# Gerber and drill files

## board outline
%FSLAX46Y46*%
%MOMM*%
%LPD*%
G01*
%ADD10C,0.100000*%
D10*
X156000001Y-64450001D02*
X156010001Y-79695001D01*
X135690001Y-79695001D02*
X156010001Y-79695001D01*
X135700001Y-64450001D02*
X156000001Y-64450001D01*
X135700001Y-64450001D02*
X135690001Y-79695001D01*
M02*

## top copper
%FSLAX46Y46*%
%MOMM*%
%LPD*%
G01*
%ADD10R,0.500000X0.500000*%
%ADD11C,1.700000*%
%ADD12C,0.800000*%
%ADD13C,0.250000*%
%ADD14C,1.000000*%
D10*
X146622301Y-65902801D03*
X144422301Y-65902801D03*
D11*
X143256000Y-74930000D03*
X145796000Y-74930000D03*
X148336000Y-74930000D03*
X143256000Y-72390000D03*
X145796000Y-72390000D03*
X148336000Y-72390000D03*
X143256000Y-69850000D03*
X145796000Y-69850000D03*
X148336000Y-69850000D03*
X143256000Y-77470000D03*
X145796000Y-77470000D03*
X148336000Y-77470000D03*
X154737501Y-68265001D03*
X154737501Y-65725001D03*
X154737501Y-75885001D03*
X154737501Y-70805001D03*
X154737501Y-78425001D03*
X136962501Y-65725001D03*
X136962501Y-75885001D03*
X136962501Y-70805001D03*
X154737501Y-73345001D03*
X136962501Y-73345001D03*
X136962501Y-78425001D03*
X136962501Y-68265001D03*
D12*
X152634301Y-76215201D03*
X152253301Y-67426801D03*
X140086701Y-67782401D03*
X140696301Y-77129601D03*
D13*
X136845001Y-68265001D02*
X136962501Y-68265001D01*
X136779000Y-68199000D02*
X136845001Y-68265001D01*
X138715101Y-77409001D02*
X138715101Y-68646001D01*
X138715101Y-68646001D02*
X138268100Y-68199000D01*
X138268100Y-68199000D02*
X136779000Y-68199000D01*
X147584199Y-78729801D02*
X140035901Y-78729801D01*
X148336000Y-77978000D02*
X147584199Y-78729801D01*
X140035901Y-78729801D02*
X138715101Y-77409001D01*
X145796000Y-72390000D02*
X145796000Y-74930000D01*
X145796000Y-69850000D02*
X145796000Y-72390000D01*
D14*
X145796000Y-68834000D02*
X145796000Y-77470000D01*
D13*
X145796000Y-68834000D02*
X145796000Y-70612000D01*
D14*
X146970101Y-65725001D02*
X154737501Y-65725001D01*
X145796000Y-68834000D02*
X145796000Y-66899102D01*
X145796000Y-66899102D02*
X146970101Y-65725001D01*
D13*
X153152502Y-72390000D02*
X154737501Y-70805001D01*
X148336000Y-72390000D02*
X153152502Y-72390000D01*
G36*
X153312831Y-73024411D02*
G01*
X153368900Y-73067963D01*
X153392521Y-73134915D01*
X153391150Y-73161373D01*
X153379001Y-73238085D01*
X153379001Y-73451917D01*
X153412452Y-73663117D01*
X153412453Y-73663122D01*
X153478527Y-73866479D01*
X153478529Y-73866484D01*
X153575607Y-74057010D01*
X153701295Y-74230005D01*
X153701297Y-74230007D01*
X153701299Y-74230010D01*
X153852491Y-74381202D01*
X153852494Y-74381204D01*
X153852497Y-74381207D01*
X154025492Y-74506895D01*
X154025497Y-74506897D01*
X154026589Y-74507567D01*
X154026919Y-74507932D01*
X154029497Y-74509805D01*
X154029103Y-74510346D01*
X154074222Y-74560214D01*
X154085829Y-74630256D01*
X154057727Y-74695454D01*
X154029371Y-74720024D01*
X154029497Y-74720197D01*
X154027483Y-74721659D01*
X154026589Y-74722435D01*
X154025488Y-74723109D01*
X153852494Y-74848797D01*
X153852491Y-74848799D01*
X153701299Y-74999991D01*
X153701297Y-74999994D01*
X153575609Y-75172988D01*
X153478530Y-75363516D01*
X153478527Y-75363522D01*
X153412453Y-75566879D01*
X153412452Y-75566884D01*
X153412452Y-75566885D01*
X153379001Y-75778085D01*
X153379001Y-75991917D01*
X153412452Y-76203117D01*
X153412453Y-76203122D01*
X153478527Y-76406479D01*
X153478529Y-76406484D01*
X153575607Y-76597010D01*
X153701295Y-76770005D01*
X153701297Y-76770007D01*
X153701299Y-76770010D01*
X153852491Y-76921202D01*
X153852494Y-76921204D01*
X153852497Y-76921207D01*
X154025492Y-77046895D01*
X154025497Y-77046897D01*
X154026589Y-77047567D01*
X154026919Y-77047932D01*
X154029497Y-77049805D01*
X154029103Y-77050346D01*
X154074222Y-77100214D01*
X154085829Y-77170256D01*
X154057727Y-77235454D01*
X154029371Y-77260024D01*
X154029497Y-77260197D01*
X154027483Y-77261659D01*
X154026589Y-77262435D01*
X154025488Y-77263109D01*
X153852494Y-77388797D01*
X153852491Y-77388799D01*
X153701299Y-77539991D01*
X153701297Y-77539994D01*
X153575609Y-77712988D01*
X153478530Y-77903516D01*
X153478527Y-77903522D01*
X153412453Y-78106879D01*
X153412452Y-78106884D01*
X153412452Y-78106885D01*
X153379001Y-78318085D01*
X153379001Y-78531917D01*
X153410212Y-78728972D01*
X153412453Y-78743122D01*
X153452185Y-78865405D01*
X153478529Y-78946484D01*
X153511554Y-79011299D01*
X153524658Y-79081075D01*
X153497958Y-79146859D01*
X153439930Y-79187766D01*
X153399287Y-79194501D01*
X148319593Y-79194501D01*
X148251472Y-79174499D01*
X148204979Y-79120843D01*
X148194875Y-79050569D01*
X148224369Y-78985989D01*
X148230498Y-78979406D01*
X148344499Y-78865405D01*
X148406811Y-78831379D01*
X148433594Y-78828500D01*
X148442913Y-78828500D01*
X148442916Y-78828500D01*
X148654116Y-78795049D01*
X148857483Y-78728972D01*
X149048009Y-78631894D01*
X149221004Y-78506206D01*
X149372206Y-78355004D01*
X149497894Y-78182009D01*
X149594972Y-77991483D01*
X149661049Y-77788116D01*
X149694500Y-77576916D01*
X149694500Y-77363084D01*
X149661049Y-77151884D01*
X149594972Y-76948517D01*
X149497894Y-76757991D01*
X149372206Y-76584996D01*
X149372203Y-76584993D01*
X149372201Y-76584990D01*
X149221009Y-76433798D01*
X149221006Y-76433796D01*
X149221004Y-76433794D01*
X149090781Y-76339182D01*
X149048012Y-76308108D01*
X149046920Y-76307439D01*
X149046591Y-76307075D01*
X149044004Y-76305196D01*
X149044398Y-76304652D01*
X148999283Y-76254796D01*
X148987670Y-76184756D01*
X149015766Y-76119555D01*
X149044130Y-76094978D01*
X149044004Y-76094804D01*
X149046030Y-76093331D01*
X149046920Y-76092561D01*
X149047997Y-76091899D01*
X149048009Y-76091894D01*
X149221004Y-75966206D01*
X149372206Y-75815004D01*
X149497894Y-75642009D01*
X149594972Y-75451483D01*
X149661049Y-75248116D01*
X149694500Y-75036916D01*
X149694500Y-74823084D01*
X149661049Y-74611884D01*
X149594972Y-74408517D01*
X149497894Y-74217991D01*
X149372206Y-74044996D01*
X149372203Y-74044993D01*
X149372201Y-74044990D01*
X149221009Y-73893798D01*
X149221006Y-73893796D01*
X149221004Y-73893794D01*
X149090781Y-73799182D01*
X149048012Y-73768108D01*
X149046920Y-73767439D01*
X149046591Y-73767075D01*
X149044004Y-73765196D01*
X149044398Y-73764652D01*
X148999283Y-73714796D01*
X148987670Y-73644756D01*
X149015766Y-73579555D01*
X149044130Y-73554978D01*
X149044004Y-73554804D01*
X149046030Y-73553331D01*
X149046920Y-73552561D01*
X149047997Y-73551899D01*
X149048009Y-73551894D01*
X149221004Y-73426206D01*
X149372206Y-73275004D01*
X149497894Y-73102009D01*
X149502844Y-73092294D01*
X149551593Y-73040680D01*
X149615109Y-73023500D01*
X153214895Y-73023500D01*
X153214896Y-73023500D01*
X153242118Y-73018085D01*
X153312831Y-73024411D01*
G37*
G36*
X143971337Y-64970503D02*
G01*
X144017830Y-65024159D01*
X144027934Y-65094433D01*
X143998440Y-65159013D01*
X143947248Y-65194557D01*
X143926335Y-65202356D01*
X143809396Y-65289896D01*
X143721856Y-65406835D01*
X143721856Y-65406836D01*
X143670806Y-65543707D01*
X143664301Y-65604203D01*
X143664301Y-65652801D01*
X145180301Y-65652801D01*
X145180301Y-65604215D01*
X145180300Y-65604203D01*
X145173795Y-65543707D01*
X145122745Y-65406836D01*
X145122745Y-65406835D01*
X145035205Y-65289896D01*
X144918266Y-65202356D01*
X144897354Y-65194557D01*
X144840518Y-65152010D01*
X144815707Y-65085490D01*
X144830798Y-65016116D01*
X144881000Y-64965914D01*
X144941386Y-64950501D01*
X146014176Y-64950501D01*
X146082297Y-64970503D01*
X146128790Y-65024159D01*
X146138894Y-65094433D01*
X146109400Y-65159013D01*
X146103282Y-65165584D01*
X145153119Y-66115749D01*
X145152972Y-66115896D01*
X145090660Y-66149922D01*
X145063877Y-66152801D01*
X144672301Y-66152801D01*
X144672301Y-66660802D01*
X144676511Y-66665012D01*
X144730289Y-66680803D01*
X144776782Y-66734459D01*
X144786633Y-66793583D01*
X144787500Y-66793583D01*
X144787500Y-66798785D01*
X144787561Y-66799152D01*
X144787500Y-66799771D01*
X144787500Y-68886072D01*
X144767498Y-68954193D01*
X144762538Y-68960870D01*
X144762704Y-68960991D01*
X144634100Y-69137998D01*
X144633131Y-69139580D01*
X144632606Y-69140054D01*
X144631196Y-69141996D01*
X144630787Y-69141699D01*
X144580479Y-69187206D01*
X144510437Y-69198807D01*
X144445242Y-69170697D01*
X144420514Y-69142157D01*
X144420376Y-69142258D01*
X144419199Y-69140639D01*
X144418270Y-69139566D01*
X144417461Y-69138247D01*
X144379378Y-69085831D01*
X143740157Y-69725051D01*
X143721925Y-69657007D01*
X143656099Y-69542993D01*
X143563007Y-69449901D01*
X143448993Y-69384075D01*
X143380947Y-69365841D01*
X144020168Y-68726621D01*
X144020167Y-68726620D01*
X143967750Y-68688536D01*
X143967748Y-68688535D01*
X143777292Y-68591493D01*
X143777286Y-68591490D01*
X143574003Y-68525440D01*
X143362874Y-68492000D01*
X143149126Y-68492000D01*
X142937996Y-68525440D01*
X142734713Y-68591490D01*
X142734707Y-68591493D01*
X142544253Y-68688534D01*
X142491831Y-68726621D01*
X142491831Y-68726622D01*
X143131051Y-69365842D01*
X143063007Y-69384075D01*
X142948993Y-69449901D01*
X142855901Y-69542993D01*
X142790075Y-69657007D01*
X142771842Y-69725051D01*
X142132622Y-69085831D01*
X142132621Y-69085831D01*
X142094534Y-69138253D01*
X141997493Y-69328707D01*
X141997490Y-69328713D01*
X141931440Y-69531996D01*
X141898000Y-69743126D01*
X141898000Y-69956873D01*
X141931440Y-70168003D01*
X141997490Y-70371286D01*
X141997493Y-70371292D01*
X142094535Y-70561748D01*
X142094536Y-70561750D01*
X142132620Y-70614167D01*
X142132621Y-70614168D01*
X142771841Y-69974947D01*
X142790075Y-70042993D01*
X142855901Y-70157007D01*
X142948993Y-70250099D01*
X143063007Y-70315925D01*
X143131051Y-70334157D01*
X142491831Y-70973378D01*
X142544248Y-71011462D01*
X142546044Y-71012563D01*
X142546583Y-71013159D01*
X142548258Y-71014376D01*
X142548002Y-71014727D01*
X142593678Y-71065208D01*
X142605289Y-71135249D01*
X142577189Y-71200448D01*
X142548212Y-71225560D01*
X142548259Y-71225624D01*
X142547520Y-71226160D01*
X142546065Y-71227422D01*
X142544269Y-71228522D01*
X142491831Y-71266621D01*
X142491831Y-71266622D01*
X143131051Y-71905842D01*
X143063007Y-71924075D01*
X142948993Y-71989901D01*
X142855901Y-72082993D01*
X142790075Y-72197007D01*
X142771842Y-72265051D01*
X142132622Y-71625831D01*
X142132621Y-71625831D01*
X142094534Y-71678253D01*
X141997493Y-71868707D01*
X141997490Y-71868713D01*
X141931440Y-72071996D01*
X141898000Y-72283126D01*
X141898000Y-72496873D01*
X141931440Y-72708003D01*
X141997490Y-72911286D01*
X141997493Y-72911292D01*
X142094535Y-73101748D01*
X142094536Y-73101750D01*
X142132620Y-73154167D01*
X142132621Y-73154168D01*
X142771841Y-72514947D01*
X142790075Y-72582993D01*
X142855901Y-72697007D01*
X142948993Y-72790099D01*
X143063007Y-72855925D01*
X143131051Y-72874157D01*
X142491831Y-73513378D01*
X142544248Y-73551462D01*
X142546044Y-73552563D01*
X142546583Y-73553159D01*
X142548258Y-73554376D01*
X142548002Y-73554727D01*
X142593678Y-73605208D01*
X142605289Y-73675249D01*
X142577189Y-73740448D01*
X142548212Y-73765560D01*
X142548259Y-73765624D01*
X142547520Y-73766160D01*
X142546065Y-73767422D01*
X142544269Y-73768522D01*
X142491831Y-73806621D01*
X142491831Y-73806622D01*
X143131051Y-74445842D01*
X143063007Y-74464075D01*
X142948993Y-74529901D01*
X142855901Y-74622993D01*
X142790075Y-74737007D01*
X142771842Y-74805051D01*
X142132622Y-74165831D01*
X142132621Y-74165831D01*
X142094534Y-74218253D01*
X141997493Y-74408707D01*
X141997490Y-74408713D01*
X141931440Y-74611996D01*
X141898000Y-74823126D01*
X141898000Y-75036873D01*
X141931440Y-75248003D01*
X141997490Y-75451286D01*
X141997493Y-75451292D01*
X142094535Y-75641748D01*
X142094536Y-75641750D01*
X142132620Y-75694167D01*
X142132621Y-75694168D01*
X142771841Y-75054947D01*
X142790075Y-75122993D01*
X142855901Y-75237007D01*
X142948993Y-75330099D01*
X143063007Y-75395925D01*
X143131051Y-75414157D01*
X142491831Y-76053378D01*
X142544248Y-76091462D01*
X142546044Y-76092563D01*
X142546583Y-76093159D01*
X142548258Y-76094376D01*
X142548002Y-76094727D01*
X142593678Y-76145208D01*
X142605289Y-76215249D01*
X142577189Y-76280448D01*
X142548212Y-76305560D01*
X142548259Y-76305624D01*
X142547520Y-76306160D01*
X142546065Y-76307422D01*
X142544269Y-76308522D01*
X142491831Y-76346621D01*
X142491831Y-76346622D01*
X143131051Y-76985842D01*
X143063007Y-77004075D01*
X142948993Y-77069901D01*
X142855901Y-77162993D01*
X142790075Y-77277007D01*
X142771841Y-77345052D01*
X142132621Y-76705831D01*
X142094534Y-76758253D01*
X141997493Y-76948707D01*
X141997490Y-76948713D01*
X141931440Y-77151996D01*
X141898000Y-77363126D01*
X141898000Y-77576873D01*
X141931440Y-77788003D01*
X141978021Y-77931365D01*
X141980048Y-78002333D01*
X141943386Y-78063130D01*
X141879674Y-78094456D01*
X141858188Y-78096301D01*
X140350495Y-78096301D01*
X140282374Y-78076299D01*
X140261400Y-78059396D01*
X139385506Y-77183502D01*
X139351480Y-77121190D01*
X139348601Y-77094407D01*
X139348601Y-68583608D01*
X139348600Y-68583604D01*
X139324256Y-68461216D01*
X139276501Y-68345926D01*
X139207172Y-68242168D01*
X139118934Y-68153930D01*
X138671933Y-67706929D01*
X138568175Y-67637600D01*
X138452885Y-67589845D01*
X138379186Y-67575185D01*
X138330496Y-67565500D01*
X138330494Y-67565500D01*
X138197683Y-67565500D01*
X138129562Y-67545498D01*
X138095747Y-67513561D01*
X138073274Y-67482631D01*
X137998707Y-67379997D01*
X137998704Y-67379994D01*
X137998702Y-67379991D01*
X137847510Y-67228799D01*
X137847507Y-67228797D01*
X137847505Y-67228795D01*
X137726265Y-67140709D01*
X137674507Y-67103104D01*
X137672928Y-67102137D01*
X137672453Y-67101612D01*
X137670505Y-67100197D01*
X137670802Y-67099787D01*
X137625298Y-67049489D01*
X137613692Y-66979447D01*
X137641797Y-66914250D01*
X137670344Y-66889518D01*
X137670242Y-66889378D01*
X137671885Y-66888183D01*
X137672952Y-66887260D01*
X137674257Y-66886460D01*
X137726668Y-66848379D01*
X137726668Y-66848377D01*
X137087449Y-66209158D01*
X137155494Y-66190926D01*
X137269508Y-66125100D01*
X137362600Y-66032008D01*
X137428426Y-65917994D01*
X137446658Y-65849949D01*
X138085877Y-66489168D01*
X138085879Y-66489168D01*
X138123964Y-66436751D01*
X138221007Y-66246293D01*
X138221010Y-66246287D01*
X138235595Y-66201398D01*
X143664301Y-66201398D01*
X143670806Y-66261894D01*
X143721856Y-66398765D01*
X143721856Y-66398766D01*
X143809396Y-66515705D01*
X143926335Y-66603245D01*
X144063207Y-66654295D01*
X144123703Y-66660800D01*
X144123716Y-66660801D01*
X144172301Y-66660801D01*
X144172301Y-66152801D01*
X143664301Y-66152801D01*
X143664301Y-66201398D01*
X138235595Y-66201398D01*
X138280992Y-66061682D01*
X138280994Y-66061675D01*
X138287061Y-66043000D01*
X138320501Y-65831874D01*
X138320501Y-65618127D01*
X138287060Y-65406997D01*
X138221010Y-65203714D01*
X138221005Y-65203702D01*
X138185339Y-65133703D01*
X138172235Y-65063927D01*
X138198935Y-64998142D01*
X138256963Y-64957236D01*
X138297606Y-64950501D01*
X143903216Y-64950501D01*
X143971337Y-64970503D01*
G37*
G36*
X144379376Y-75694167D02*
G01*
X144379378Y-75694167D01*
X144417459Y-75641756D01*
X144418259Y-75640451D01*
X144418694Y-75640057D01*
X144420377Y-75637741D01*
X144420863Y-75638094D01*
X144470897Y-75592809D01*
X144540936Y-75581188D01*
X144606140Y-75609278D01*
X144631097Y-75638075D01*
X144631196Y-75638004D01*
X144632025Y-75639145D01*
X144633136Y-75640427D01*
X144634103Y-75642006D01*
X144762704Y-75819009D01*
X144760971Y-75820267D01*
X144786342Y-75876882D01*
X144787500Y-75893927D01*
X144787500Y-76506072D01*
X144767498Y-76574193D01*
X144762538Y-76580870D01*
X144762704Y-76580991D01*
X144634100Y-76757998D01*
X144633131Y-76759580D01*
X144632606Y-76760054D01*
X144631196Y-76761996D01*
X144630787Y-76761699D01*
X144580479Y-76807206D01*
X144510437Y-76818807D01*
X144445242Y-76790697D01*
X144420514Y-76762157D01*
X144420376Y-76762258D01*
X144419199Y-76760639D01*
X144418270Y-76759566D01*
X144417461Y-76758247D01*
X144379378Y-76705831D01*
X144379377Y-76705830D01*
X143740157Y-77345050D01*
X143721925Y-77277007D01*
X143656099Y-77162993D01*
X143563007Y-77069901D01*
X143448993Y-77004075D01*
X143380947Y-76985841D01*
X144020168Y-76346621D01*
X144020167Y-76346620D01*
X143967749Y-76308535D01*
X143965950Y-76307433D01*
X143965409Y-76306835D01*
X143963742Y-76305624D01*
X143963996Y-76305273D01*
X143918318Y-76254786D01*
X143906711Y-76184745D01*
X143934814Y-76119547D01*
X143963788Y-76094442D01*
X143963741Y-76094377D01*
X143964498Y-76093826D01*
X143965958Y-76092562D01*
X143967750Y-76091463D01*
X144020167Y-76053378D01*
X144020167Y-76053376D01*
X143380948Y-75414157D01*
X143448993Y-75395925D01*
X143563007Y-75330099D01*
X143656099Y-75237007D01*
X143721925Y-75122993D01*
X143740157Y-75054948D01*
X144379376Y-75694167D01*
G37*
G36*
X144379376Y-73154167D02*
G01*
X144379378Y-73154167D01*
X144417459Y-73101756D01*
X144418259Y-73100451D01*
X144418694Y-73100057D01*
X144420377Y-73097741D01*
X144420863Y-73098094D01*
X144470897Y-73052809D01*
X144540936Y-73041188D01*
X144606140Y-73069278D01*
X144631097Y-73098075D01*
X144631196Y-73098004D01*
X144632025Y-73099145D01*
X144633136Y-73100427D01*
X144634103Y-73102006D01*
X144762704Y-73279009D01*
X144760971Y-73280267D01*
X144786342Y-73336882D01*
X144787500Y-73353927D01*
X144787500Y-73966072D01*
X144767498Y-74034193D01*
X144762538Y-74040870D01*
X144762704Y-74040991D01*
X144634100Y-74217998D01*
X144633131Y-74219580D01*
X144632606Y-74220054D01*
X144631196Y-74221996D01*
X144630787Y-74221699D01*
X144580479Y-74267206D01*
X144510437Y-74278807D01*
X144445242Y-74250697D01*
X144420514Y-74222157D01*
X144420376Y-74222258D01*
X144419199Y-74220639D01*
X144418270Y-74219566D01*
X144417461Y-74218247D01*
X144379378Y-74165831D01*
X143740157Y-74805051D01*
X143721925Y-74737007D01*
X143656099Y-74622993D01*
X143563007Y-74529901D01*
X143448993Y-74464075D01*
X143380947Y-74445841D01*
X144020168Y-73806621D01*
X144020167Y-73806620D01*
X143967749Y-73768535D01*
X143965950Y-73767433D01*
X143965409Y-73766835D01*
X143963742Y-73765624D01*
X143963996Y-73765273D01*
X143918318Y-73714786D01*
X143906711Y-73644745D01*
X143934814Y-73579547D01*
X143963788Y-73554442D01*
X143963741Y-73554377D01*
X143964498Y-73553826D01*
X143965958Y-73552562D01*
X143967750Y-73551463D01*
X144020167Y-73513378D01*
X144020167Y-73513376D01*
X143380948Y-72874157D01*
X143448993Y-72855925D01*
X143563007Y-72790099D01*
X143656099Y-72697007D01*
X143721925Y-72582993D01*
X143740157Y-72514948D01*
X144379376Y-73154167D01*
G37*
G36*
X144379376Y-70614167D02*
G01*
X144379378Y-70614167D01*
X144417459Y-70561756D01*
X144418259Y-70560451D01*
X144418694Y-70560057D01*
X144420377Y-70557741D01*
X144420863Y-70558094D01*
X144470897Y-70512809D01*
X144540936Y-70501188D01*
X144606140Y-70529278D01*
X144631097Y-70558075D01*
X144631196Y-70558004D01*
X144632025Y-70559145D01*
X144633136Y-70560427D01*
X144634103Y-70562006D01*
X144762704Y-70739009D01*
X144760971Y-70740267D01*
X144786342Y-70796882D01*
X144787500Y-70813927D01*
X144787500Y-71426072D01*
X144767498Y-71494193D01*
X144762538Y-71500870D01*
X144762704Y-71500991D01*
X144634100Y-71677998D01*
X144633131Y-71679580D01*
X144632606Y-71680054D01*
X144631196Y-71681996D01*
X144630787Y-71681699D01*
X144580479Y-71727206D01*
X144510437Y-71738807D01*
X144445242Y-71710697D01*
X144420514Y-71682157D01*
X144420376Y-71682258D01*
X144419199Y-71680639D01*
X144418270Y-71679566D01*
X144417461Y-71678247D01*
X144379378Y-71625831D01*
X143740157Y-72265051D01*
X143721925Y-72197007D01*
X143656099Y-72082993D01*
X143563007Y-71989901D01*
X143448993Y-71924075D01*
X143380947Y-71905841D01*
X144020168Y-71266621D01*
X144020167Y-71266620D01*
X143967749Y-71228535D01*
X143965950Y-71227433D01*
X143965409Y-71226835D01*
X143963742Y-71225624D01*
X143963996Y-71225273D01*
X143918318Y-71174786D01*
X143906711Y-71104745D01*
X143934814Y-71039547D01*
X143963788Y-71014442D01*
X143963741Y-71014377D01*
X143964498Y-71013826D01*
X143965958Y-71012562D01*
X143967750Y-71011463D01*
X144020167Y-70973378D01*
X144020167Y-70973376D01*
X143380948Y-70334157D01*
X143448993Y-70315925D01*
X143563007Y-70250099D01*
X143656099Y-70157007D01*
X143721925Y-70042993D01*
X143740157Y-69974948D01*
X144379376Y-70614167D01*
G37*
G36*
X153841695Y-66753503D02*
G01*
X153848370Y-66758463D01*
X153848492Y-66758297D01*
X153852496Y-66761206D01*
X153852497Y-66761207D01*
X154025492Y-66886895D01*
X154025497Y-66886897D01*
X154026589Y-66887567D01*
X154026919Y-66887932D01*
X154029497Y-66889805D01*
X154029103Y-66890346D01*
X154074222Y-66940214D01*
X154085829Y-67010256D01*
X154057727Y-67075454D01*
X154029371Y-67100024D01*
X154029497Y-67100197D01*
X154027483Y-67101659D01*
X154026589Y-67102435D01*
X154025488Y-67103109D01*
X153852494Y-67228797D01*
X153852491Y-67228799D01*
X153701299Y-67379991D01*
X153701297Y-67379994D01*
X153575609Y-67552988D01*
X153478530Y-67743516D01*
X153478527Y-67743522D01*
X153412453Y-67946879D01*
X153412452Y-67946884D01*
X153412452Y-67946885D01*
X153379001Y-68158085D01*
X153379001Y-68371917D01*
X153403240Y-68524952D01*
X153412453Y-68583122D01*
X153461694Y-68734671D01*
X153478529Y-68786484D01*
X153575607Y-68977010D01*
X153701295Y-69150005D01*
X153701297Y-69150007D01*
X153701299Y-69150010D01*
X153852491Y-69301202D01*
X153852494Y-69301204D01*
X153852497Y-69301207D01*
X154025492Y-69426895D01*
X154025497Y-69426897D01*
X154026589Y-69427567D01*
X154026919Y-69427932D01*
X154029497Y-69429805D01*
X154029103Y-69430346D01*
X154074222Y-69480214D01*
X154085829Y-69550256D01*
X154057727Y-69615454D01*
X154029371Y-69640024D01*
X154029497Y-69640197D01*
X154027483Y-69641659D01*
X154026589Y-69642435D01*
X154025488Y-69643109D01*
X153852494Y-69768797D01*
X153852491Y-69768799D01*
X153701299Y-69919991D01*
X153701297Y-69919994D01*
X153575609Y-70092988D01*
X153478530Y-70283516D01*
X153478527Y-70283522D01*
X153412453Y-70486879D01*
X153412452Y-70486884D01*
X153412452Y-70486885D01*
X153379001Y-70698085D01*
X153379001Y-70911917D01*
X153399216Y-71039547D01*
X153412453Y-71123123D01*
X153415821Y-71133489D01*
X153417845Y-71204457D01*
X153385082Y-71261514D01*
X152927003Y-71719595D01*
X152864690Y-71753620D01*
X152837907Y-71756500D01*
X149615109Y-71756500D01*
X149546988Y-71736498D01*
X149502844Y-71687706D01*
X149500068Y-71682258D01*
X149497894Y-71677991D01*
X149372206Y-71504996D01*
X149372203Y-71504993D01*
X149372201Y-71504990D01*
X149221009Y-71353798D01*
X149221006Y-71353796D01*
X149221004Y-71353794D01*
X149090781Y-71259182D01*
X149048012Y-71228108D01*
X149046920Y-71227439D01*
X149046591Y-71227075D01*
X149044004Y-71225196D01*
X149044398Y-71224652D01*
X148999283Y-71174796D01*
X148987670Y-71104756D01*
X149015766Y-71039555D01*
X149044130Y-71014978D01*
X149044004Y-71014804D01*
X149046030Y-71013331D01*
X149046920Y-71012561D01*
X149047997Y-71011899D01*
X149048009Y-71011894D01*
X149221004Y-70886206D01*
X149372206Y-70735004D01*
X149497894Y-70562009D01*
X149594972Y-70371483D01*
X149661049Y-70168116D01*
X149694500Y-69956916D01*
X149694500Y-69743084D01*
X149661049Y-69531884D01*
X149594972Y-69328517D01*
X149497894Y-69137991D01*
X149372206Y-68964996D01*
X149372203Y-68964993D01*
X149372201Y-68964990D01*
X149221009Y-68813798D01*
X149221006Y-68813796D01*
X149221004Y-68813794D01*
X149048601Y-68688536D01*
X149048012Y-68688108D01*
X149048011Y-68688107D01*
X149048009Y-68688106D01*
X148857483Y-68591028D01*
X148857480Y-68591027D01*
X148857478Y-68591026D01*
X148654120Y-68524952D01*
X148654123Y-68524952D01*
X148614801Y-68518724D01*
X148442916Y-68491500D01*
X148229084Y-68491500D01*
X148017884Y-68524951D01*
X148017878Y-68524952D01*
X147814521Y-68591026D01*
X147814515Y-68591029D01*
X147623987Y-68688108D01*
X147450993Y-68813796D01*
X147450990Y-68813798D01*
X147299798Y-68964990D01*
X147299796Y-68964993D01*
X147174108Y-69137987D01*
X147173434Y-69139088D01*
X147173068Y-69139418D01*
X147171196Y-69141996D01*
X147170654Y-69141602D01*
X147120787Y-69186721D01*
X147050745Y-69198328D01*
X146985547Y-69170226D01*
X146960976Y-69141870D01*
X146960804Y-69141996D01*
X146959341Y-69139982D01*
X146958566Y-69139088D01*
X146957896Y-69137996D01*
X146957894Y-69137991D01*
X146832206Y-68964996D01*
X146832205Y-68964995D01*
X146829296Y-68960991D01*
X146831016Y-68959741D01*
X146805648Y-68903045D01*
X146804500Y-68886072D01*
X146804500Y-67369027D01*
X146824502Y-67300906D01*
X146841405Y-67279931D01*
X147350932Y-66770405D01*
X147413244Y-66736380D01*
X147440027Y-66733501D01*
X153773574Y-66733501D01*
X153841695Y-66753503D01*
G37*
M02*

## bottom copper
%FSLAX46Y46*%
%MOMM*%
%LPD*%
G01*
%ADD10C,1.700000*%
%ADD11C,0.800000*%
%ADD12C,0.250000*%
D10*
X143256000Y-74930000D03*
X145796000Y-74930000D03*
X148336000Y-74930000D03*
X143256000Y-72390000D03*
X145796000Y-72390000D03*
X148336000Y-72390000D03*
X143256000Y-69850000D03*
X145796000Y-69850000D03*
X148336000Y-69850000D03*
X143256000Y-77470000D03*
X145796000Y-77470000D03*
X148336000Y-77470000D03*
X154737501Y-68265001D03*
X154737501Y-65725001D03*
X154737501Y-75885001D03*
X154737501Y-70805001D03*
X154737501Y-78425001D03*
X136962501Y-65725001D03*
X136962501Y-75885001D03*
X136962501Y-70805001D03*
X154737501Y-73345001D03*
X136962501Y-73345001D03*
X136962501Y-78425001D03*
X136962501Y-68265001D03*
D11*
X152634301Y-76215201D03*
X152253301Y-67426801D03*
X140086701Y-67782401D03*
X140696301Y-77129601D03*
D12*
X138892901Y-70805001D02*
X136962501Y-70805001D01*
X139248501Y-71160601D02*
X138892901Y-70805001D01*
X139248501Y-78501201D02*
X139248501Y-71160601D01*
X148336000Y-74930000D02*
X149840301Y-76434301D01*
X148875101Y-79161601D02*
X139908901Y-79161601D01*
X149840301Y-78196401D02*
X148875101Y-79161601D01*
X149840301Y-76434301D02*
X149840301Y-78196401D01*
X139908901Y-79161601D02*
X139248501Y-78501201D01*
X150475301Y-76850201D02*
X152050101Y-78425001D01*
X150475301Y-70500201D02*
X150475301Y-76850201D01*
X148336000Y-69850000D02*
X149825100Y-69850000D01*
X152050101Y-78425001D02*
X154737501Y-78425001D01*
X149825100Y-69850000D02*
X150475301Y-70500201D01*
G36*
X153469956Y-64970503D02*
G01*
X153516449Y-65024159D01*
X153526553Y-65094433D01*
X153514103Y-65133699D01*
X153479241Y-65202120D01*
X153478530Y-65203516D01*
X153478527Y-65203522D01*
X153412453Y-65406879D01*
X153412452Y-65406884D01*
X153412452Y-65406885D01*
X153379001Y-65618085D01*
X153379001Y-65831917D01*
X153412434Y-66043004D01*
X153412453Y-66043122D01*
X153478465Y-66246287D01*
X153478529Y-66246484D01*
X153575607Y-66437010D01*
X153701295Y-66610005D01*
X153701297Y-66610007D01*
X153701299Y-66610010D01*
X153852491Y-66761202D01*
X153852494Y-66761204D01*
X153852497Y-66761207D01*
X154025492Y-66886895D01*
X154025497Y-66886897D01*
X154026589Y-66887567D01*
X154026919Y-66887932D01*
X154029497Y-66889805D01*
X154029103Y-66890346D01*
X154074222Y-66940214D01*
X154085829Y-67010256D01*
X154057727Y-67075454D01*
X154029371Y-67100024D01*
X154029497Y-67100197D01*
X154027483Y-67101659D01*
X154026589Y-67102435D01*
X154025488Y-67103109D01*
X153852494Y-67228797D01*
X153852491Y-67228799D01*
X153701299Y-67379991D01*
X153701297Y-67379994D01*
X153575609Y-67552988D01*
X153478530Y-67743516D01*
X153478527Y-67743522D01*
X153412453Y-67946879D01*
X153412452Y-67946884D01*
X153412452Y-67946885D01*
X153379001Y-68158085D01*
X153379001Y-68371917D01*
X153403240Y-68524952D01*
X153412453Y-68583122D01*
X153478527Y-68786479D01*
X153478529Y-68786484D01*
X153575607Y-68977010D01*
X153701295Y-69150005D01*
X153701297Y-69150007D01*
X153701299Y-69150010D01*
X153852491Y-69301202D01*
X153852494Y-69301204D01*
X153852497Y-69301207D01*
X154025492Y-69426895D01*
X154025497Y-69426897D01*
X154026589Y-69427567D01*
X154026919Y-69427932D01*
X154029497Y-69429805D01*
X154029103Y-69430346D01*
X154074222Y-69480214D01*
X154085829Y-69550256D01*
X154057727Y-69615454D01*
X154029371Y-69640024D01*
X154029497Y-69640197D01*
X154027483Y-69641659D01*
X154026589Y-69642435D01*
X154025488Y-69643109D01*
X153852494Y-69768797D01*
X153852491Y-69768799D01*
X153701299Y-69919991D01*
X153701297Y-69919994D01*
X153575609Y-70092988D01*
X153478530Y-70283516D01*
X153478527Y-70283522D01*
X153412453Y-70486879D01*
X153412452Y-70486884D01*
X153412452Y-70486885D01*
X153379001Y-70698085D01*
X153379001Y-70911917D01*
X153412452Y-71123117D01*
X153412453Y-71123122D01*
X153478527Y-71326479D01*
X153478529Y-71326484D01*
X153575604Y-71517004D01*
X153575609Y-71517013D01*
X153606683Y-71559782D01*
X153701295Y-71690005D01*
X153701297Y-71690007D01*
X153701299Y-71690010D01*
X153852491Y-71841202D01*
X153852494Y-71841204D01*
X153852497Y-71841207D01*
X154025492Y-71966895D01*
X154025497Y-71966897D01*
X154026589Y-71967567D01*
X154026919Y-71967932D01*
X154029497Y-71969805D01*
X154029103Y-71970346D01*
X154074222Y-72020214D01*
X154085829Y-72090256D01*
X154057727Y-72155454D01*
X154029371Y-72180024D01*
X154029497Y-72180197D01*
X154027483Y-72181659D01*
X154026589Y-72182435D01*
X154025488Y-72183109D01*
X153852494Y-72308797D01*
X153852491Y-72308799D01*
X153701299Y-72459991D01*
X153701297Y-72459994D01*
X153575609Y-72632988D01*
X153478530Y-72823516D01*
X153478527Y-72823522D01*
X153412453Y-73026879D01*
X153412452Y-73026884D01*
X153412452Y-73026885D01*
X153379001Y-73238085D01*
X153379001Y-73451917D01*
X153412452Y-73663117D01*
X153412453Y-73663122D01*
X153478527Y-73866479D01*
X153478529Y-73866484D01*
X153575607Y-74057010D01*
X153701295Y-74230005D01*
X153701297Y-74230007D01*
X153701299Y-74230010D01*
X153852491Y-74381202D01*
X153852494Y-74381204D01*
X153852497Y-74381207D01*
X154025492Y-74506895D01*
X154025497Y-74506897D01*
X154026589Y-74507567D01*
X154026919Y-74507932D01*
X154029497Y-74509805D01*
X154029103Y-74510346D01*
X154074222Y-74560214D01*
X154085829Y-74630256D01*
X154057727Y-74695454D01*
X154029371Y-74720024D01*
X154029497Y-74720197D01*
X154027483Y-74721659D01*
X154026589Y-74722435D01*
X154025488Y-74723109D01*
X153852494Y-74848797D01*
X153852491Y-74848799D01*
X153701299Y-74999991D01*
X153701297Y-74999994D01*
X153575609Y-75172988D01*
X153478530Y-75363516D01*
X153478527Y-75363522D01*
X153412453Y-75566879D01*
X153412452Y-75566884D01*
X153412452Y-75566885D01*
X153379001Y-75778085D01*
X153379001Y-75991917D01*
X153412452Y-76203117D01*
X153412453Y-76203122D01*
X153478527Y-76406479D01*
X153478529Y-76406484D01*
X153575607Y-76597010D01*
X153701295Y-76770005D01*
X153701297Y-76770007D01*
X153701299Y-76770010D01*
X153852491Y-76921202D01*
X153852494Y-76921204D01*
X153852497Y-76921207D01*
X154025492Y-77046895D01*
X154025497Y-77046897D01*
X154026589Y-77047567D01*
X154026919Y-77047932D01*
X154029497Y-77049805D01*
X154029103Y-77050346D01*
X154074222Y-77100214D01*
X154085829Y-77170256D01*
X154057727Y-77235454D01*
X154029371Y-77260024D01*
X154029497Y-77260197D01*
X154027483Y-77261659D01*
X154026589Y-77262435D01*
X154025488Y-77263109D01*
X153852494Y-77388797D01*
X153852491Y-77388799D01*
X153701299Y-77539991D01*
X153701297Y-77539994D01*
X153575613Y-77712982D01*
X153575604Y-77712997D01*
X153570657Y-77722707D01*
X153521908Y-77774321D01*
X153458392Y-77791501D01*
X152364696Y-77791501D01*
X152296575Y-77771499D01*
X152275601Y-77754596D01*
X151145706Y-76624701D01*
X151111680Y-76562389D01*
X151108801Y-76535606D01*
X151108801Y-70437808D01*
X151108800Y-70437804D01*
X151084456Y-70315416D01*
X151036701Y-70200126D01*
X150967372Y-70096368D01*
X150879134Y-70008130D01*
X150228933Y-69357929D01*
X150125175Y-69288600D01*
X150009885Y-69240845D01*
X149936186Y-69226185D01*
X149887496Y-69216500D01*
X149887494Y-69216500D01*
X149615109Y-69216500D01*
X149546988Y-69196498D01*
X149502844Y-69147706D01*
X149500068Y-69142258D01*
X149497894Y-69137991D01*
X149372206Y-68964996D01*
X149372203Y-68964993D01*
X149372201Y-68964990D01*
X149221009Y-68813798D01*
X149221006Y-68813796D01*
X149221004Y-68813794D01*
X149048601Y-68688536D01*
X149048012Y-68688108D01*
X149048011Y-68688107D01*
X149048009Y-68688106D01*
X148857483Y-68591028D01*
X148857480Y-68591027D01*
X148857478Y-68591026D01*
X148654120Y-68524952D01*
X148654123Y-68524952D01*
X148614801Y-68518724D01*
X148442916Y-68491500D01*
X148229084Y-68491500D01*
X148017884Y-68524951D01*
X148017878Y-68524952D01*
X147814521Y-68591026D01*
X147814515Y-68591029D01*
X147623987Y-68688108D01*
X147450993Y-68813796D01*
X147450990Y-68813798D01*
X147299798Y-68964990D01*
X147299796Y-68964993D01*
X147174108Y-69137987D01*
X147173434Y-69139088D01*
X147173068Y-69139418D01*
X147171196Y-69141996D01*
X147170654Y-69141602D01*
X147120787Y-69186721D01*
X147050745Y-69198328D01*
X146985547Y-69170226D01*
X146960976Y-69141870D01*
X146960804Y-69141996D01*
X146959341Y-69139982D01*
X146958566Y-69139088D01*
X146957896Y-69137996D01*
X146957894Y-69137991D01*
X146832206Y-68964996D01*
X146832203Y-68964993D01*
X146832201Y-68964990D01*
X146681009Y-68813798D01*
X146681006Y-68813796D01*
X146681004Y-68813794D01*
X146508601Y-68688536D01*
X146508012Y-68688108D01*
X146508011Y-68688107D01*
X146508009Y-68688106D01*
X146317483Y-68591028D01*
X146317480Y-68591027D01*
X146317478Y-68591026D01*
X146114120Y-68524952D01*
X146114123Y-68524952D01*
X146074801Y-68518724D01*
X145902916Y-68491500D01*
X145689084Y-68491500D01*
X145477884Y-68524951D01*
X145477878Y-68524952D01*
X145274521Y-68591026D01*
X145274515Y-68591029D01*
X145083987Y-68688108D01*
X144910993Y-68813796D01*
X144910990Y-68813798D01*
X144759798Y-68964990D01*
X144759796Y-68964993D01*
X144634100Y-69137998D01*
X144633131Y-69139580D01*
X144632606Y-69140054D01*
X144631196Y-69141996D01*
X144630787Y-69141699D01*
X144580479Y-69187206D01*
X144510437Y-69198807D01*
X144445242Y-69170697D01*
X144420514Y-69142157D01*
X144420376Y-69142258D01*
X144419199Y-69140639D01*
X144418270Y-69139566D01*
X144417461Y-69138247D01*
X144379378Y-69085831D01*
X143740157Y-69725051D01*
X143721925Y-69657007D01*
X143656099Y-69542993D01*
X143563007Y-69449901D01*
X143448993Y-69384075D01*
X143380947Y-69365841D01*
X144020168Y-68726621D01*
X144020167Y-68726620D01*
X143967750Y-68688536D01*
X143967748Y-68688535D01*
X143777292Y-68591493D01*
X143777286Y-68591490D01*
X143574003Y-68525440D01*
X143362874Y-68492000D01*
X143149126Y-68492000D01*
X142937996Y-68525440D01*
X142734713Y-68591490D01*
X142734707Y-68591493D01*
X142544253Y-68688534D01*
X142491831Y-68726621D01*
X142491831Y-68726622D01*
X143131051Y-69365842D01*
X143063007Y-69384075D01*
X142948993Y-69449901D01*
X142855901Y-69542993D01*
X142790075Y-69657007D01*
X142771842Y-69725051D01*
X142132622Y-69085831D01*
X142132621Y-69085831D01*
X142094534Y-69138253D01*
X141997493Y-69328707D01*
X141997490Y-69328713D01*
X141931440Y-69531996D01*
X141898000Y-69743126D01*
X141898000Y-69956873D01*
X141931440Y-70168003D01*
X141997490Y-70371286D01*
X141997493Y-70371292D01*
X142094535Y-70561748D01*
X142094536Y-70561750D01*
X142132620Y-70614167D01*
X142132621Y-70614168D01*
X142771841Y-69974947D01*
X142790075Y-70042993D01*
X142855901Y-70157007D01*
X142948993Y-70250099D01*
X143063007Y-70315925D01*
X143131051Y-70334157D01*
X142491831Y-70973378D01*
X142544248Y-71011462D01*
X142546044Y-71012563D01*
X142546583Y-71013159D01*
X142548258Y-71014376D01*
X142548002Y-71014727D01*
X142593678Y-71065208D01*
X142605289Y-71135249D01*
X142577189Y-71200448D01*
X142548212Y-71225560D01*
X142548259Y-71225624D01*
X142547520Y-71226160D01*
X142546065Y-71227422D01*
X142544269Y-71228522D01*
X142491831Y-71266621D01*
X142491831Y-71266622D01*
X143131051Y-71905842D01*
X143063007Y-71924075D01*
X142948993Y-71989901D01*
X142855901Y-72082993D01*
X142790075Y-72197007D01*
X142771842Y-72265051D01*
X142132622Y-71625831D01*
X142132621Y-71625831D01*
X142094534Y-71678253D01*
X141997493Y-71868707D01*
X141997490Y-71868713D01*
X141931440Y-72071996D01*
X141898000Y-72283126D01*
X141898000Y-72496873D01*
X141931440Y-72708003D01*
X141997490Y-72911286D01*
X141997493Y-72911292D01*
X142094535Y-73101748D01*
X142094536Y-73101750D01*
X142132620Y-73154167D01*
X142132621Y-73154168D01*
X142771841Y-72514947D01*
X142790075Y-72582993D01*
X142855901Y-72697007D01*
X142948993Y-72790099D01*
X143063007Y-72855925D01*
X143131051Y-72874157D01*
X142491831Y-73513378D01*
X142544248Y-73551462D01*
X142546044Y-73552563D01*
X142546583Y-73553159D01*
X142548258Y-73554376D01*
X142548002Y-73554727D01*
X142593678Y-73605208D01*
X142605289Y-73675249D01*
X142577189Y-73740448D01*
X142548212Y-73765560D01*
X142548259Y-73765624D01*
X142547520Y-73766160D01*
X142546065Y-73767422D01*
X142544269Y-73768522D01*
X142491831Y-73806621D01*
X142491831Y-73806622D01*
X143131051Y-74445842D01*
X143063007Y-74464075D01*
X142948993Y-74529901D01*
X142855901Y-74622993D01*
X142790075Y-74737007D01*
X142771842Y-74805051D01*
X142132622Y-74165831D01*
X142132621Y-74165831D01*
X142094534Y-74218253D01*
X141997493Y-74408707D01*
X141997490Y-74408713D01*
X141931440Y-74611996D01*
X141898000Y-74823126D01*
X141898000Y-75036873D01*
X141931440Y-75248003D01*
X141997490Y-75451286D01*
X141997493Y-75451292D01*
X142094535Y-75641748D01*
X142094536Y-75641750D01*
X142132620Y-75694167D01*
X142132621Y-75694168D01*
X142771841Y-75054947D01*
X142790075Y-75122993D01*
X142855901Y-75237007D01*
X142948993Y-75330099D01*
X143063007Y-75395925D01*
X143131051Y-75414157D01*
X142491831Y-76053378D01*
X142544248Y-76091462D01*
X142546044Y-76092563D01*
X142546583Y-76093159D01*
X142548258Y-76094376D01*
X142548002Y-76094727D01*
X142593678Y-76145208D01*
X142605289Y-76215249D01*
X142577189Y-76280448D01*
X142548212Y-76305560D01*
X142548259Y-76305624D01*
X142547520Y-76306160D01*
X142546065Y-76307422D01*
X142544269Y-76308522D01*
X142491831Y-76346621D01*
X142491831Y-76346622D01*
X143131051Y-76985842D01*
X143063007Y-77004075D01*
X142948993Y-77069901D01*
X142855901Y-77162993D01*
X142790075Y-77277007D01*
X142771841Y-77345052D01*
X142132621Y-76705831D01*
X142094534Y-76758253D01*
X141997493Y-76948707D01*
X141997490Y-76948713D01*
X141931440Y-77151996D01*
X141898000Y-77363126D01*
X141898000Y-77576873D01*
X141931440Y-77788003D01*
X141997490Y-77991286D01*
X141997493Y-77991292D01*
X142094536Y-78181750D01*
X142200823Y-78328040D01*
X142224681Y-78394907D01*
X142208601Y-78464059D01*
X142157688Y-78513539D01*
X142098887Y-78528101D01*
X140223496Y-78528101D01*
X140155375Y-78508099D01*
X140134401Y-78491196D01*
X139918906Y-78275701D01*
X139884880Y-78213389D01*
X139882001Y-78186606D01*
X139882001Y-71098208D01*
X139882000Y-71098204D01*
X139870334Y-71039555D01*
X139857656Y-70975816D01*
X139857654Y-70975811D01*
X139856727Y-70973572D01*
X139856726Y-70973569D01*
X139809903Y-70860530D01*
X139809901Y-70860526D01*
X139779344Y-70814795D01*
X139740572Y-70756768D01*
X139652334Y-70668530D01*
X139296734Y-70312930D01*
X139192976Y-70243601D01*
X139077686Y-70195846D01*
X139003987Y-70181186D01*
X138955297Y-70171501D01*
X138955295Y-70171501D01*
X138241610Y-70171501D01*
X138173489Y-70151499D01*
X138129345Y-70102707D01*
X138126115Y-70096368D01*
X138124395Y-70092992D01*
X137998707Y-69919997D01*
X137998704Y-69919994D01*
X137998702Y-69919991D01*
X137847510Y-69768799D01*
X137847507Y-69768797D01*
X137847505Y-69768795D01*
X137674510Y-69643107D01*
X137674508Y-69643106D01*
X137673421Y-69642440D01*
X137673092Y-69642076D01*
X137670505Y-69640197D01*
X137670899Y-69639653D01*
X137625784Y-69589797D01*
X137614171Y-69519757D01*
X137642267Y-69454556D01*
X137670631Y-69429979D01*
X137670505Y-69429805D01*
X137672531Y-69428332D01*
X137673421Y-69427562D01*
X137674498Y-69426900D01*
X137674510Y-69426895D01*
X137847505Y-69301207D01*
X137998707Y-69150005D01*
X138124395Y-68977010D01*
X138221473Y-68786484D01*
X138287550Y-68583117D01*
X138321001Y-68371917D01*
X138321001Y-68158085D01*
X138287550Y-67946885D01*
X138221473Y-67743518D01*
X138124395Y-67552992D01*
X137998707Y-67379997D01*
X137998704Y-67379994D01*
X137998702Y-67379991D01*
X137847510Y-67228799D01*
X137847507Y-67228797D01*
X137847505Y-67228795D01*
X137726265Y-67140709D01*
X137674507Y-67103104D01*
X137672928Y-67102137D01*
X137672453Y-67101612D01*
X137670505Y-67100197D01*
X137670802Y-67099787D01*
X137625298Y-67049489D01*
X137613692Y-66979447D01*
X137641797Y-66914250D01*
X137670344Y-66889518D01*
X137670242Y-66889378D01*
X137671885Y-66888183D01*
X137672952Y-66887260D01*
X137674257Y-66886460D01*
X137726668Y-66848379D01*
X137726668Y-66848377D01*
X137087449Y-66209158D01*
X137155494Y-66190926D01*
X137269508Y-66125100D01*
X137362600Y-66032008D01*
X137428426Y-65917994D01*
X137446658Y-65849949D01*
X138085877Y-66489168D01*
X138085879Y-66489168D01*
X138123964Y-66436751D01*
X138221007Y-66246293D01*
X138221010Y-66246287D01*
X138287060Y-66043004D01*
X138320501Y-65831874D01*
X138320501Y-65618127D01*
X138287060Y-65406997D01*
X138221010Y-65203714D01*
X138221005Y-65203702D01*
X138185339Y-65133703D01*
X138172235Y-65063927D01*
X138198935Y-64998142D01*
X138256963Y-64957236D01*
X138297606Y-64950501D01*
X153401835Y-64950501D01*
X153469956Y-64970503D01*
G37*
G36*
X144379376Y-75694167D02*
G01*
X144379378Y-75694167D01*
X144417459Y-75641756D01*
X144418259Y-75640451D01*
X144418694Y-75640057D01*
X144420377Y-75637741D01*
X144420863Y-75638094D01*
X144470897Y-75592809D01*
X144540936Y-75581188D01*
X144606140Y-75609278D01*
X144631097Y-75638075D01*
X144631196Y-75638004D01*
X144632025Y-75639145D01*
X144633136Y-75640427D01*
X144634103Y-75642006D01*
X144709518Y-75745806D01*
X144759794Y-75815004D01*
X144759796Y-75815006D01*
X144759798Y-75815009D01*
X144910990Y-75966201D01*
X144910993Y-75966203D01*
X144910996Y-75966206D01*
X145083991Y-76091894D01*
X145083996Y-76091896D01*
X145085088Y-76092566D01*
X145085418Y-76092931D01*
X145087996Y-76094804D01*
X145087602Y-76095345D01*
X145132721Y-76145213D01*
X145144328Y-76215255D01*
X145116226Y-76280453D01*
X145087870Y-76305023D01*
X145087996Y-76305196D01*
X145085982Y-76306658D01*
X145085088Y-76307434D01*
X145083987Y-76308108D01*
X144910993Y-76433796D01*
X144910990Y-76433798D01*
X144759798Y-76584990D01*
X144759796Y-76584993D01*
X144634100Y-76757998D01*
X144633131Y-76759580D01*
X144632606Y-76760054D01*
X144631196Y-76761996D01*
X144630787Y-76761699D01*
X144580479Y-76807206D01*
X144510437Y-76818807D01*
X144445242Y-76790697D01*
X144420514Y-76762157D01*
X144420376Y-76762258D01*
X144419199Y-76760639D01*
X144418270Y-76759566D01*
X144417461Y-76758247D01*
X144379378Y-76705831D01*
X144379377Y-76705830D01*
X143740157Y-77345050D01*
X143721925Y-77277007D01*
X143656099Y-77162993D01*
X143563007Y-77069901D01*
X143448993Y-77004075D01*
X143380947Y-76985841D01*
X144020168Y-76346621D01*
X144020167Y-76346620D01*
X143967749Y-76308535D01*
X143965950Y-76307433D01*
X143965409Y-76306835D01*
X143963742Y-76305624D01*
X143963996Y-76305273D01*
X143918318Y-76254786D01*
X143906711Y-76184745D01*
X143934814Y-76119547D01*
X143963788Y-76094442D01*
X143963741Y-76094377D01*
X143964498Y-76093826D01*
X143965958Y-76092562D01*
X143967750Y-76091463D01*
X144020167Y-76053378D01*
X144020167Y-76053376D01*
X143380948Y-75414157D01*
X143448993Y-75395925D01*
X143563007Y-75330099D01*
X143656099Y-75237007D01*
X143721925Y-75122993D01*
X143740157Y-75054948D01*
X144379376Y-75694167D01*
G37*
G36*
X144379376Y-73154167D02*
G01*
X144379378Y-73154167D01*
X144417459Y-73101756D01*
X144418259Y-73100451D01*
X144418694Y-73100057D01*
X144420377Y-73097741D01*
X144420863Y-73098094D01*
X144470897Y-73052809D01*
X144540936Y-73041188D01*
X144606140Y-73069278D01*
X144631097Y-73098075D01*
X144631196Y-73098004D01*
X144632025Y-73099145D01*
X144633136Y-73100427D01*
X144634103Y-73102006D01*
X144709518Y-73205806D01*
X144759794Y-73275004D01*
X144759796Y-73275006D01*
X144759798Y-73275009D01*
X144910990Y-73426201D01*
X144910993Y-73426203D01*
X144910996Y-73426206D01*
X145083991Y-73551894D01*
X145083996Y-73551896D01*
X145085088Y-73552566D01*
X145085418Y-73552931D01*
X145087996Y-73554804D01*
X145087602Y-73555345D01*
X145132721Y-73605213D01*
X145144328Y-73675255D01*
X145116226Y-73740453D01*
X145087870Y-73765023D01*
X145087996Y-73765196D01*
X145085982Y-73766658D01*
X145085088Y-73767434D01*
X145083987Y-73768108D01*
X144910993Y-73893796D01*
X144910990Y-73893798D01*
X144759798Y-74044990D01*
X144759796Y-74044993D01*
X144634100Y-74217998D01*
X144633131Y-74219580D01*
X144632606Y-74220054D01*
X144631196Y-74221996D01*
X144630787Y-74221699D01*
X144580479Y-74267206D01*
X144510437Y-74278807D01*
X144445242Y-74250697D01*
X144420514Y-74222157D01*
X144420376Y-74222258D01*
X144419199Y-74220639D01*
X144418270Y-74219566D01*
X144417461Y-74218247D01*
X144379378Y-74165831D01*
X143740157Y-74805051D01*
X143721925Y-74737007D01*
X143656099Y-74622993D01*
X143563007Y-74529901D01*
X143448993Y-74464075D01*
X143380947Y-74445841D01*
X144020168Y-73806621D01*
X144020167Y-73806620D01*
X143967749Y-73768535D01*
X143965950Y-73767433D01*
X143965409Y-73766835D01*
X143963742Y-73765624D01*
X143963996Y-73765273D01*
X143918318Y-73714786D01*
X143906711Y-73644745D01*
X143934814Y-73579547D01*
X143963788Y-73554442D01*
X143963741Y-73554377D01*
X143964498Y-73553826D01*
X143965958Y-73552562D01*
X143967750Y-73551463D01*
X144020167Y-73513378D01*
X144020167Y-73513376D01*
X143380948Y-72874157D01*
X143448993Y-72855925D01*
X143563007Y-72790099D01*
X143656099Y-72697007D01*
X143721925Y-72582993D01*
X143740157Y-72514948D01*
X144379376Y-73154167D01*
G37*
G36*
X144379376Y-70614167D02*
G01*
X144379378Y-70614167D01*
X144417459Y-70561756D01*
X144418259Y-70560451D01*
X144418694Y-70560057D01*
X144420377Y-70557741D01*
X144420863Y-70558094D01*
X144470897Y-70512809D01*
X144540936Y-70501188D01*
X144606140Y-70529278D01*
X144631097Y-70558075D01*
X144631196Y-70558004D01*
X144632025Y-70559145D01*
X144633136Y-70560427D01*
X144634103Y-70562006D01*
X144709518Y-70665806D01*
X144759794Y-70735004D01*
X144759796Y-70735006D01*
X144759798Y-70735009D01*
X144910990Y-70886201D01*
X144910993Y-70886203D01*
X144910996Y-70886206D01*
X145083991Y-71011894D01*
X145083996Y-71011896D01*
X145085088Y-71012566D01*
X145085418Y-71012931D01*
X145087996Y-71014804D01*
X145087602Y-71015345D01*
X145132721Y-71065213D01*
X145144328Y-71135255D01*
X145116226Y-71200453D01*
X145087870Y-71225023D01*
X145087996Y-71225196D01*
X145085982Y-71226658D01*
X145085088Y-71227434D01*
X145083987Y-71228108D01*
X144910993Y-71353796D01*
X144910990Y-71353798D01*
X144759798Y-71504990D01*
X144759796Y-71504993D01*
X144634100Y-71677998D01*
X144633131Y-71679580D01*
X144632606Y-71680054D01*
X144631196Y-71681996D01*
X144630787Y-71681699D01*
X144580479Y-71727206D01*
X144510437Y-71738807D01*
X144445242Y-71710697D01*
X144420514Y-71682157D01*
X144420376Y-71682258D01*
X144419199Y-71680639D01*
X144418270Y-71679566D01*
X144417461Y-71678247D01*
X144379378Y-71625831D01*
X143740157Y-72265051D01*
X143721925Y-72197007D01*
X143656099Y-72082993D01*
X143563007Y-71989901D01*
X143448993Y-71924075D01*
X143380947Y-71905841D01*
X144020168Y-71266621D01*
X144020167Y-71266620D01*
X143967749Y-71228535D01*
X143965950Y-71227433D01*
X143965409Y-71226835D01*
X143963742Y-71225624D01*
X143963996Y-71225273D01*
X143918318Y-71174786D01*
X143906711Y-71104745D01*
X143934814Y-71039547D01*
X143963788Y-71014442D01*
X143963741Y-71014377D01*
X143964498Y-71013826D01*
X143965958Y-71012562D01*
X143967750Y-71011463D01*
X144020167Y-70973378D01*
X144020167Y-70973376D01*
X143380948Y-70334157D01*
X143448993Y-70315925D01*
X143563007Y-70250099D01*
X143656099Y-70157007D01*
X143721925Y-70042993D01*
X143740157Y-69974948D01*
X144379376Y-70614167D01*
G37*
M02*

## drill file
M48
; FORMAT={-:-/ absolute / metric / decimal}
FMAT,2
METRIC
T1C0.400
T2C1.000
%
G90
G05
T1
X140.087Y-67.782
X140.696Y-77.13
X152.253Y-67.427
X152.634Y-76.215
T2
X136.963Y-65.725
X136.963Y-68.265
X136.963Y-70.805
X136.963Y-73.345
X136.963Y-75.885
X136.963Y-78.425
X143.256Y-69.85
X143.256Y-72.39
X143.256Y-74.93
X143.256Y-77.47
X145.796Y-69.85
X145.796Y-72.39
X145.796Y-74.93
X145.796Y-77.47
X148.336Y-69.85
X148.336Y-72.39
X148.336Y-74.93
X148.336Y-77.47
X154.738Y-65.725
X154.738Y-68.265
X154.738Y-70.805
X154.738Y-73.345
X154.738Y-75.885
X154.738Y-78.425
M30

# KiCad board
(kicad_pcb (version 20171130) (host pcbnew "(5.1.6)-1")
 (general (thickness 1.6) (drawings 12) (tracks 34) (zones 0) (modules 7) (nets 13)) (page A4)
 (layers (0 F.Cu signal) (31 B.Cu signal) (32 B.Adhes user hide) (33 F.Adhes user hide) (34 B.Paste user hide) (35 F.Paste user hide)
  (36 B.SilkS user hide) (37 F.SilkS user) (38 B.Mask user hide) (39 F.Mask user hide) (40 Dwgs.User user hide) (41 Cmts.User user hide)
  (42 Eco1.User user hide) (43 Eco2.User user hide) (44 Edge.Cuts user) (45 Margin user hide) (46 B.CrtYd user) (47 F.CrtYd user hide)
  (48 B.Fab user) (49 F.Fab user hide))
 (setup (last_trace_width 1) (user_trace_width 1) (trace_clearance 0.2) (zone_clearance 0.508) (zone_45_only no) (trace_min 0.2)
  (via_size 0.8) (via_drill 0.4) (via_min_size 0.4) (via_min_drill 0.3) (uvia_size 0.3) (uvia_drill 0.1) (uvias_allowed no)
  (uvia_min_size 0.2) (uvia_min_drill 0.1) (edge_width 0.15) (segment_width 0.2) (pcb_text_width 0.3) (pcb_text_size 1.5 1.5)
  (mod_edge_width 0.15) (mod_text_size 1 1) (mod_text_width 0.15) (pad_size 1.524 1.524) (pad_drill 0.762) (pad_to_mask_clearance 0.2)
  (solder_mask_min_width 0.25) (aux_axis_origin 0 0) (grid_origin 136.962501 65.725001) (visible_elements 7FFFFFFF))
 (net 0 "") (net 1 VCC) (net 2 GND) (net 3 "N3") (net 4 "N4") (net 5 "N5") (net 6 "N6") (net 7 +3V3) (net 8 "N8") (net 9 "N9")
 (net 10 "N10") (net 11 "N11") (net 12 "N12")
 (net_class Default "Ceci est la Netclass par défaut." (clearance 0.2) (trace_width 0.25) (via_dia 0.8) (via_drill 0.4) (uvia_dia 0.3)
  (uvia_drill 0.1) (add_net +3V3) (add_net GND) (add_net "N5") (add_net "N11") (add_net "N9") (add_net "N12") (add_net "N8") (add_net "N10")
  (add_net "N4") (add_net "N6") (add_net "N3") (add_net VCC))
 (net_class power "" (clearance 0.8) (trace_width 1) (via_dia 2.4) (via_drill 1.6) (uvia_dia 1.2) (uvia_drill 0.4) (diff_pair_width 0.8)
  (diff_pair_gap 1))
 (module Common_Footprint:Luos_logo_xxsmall (layer F.Cu) (at 141.331301 66.182201)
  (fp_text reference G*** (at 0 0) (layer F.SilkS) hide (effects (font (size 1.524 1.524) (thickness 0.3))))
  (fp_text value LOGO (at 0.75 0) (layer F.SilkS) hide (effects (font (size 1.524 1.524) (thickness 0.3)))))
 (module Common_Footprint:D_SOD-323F (layer F.Cu) (at 145.522301 65.902801 180)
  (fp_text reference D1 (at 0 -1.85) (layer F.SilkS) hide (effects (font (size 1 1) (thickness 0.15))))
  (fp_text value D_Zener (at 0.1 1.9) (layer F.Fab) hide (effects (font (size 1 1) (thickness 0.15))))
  (pad 1 smd rect (at -1.1 0 180) (size 0.5 0.5) (layers F.Cu F.Paste F.Mask) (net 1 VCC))
  (pad 2 smd rect (at 1.1 0 180) (size 0.5 0.5) (layers F.Cu F.Paste F.Mask) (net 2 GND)))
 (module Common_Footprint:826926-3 (layer F.Cu) (at 145.796 74.93 180)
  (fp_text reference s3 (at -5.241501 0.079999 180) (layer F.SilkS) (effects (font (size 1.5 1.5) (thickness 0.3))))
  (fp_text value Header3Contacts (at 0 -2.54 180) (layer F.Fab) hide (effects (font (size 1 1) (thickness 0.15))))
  (pad 3 thru_hole circle (at 2.54 0 180) (size 1.7 1.7) (drill 1) (layers *.Cu *.Mask) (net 2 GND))
  (pad 2 thru_hole circle (at 0 0 180) (size 1.7 1.7) (drill 1) (layers *.Cu *.Mask) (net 1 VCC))
  (pad 1 thru_hole circle (at -2.54 0 180) (size 1.7 1.7) (drill 1) (layers *.Cu *.Mask) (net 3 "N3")))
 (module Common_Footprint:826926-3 (layer F.Cu) (at 145.796 72.39 180)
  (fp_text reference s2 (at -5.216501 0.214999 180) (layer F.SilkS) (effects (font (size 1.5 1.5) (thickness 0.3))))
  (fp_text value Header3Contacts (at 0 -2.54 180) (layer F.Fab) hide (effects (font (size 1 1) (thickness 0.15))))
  (pad 3 thru_hole circle (at 2.54 0 180) (size 1.7 1.7) (drill 1) (layers *.Cu *.Mask) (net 2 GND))
  (pad 2 thru_hole circle (at 0 0 180) (size 1.7 1.7) (drill 1) (layers *.Cu *.Mask) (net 1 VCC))
  (pad 1 thru_hole circle (at -2.54 0 180) (size 1.7 1.7) (drill 1) (layers *.Cu *.Mask) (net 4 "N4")))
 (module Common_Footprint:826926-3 (layer F.Cu) (at 145.796 69.85 180)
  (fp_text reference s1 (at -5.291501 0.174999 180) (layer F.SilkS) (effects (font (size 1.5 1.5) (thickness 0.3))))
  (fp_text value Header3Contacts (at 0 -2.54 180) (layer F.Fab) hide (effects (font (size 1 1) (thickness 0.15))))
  (pad 3 thru_hole circle (at 2.54 0 180) (size 1.7 1.7) (drill 1) (layers *.Cu *.Mask) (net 2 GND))
  (pad 2 thru_hole circle (at 0 0 180) (size 1.7 1.7) (drill 1) (layers *.Cu *.Mask) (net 1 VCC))
  (pad 1 thru_hole circle (at -2.54 0 180) (size 1.7 1.7) (drill 1) (layers *.Cu *.Mask) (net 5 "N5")))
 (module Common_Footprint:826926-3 (layer F.Cu) (at 145.796 77.47 180)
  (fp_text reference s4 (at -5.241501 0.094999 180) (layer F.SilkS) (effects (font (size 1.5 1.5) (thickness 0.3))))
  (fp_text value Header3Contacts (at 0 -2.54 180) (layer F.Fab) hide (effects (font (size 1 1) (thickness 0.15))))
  (pad 3 thru_hole circle (at 2.54 0 180) (size 1.7 1.7) (drill 1) (layers *.Cu *.Mask) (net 2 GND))
  (pad 2 thru_hole circle (at 0 0 180) (size 1.7 1.7) (drill 1) (layers *.Cu *.Mask) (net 1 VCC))
  (pad 1 thru_hole circle (at -2.54 0 180) (size 1.7 1.7) (drill 1) (layers *.Cu *.Mask) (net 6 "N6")))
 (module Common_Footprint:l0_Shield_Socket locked (layer F.Cu) (at 145.850001 72.075001)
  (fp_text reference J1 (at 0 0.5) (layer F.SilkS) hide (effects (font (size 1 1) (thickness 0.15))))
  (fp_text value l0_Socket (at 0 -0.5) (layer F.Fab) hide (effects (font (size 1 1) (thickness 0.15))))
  (fp_line (start 10.15 -7.625) (end 10.16 7.62) (layer Edge.Cuts) (width 0.1))
  (fp_line (start -10.16 7.62) (end 10.16 7.62) (layer Edge.Cuts) (width 0.1))
  (fp_line (start -10.15 -7.625) (end 10.15 -7.625) (layer Edge.Cuts) (width 0.1))
  (fp_line (start -10.15 -7.625) (end -10.16 7.62) (layer Edge.Cuts) (width 0.1))
  (pad 5 thru_hole circle (at 8.8875 -3.81 270) (size 1.7 1.7) (drill 1) (layers *.Cu *.Mask) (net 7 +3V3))
  (pad 6 thru_hole circle (at 8.8875 -6.35 270) (size 1.7 1.7) (drill 1) (layers *.Cu *.Mask) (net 1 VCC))
  (pad 2 thru_hole circle (at 8.8875 3.81 270) (size 1.7 1.7) (drill 1) (layers *.Cu *.Mask) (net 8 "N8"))
  (pad 4 thru_hole circle (at 8.8875 -1.27 270) (size 1.7 1.7) (drill 1) (layers *.Cu *.Mask) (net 4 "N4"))
  (pad 1 thru_hole circle (at 8.8875 6.35 270) (size 1.7 1.7) (drill 1) (layers *.Cu *.Mask) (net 5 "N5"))
  (pad 7 thru_hole circle (at -8.8875 -6.35 270) (size 1.7 1.7) (drill 1) (layers *.Cu *.Mask) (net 2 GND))
  (pad 11 thru_hole circle (at -8.8875 3.81 270) (size 1.7 1.7) (drill 1) (layers *.Cu *.Mask) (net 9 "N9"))
  (pad 9 thru_hole circle (at -8.8875 -1.27 270) (size 1.7 1.7) (drill 1) (layers *.Cu *.Mask) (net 3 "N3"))
  (pad 3 thru_hole circle (at 8.8875 1.27 270) (size 1.7 1.7) (drill 1) (layers *.Cu *.Mask) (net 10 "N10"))
  (pad 10 thru_hole circle (at -8.8875 1.27 270) (size 1.7 1.7) (drill 1) (layers *.Cu *.Mask) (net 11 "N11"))
  (pad 12 thru_hole circle (at -8.8875 6.35 270) (size 1.7 1.7) (drill 1) (layers *.Cu *.Mask) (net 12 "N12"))
  (pad 8 thru_hole circle (at -8.8875 -3.81 270) (size 1.7 1.7) (drill 1) (layers *.Cu *.Mask) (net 6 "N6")))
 (segment (start 136.845001 68.265001) (end 136.962501 68.265001) (width 0.25) (layer F.Cu) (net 6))
 (segment (start 136.779 68.199) (end 136.845001 68.265001) (width 0.25) (layer F.Cu) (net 6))
 (segment (start 138.715101 77.409001) (end 138.715101 68.646001) (width 0.25) (layer F.Cu) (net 6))
 (segment (start 138.715101 68.646001) (end 138.2681 68.199) (width 0.25) (layer F.Cu) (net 6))
 (segment (start 138.2681 68.199) (end 136.779 68.199) (width 0.25) (layer F.Cu) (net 6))
 (segment (start 147.584199 78.729801) (end 140.035901 78.729801) (width 0.25) (layer F.Cu) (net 6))
 (segment (start 148.336 77.978) (end 147.584199 78.729801) (width 0.25) (layer F.Cu) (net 6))
 (segment (start 140.035901 78.729801) (end 138.715101 77.409001) (width 0.25) (layer F.Cu) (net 6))
 (segment (start 138.892901 70.805001) (end 136.962501 70.805001) (width 0.25) (layer B.Cu) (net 3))
 (segment (start 139.248501 71.160601) (end 138.892901 70.805001) (width 0.25) (layer B.Cu) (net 3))
 (segment (start 139.248501 78.501201) (end 139.248501 71.160601) (width 0.25) (layer B.Cu) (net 3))
 (segment (start 148.336 74.93) (end 149.840301 76.434301) (width 0.25) (layer B.Cu) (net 3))
 (segment (start 148.875101 79.161601) (end 139.908901 79.161601) (width 0.25) (layer B.Cu) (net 3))
 (segment (start 149.840301 78.196401) (end 148.875101 79.161601) (width 0.25) (layer B.Cu) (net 3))
 (segment (start 149.840301 76.434301) (end 149.840301 78.196401) (width 0.25) (layer B.Cu) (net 3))
 (segment (start 139.908901 79.161601) (end 139.248501 78.501201) (width 0.25) (layer B.Cu) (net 3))
 (via (at 152.634301 76.215201) (size 0.8) (drill 0.4) (layers F.Cu B.Cu) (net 2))
 (via (at 152.253301 67.426801) (size 0.8) (drill 0.4) (layers F.Cu B.Cu) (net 2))
 (via (at 140.086701 67.782401) (size 0.8) (drill 0.4) (layers F.Cu B.Cu) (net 2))
 (via (at 140.696301 77.129601) (size 0.8) (drill 0.4) (layers F.Cu B.Cu) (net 2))
 (segment (start 150.475301 76.850201) (end 152.050101 78.425001) (width 0.25) (layer B.Cu) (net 5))
 (segment (start 150.475301 70.500201) (end 150.475301 76.850201) (width 0.25) (layer B.Cu) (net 5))
 (segment (start 148.336 69.85) (end 149.8251 69.85) (width 0.25) (layer B.Cu) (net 5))
 (segment (start 152.050101 78.425001) (end 154.737501 78.425001) (width 0.25) (layer B.Cu) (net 5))
 (segment (start 149.8251 69.85) (end 150.475301 70.500201) (width 0.25) (layer B.Cu) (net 5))
 (segment (start 145.796 72.39) (end 145.796 74.93) (width 0.25) (layer F.Cu) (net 1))
 (segment (start 145.796 69.85) (end 145.796 72.39) (width 0.25) (layer F.Cu) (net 1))
 (segment (start 145.796 68.834) (end 145.796 77.47) (width 1) (layer F.Cu) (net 1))
 (segment (start 145.796 68.834) (end 145.796 70.612) (width 0.25) (layer F.Cu) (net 1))
 (segment (start 146.970101 65.725001) (end 154.737501 65.725001) (width 1) (layer F.Cu) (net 1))
 (segment (start 145.796 68.834) (end 145.796 66.899102) (width 1) (layer F.Cu) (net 1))
 (segment (start 145.796 66.899102) (end 146.970101 65.725001) (width 1) (layer F.Cu) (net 1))
 (segment (start 153.152502 72.39) (end 154.737501 70.805001) (width 0.25) (layer F.Cu) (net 4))
 (segment (start 148.336 72.39) (end 153.152502 72.39) (width 0.25) (layer F.Cu) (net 4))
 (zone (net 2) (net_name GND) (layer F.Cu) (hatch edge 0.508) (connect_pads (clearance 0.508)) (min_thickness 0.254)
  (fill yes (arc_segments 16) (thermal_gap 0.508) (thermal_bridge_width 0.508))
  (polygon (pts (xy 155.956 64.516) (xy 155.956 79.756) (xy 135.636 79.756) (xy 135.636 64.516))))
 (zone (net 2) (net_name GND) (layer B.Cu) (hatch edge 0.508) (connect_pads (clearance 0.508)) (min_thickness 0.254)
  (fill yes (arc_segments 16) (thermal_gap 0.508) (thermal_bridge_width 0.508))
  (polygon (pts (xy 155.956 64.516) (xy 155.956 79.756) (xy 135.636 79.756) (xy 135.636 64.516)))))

